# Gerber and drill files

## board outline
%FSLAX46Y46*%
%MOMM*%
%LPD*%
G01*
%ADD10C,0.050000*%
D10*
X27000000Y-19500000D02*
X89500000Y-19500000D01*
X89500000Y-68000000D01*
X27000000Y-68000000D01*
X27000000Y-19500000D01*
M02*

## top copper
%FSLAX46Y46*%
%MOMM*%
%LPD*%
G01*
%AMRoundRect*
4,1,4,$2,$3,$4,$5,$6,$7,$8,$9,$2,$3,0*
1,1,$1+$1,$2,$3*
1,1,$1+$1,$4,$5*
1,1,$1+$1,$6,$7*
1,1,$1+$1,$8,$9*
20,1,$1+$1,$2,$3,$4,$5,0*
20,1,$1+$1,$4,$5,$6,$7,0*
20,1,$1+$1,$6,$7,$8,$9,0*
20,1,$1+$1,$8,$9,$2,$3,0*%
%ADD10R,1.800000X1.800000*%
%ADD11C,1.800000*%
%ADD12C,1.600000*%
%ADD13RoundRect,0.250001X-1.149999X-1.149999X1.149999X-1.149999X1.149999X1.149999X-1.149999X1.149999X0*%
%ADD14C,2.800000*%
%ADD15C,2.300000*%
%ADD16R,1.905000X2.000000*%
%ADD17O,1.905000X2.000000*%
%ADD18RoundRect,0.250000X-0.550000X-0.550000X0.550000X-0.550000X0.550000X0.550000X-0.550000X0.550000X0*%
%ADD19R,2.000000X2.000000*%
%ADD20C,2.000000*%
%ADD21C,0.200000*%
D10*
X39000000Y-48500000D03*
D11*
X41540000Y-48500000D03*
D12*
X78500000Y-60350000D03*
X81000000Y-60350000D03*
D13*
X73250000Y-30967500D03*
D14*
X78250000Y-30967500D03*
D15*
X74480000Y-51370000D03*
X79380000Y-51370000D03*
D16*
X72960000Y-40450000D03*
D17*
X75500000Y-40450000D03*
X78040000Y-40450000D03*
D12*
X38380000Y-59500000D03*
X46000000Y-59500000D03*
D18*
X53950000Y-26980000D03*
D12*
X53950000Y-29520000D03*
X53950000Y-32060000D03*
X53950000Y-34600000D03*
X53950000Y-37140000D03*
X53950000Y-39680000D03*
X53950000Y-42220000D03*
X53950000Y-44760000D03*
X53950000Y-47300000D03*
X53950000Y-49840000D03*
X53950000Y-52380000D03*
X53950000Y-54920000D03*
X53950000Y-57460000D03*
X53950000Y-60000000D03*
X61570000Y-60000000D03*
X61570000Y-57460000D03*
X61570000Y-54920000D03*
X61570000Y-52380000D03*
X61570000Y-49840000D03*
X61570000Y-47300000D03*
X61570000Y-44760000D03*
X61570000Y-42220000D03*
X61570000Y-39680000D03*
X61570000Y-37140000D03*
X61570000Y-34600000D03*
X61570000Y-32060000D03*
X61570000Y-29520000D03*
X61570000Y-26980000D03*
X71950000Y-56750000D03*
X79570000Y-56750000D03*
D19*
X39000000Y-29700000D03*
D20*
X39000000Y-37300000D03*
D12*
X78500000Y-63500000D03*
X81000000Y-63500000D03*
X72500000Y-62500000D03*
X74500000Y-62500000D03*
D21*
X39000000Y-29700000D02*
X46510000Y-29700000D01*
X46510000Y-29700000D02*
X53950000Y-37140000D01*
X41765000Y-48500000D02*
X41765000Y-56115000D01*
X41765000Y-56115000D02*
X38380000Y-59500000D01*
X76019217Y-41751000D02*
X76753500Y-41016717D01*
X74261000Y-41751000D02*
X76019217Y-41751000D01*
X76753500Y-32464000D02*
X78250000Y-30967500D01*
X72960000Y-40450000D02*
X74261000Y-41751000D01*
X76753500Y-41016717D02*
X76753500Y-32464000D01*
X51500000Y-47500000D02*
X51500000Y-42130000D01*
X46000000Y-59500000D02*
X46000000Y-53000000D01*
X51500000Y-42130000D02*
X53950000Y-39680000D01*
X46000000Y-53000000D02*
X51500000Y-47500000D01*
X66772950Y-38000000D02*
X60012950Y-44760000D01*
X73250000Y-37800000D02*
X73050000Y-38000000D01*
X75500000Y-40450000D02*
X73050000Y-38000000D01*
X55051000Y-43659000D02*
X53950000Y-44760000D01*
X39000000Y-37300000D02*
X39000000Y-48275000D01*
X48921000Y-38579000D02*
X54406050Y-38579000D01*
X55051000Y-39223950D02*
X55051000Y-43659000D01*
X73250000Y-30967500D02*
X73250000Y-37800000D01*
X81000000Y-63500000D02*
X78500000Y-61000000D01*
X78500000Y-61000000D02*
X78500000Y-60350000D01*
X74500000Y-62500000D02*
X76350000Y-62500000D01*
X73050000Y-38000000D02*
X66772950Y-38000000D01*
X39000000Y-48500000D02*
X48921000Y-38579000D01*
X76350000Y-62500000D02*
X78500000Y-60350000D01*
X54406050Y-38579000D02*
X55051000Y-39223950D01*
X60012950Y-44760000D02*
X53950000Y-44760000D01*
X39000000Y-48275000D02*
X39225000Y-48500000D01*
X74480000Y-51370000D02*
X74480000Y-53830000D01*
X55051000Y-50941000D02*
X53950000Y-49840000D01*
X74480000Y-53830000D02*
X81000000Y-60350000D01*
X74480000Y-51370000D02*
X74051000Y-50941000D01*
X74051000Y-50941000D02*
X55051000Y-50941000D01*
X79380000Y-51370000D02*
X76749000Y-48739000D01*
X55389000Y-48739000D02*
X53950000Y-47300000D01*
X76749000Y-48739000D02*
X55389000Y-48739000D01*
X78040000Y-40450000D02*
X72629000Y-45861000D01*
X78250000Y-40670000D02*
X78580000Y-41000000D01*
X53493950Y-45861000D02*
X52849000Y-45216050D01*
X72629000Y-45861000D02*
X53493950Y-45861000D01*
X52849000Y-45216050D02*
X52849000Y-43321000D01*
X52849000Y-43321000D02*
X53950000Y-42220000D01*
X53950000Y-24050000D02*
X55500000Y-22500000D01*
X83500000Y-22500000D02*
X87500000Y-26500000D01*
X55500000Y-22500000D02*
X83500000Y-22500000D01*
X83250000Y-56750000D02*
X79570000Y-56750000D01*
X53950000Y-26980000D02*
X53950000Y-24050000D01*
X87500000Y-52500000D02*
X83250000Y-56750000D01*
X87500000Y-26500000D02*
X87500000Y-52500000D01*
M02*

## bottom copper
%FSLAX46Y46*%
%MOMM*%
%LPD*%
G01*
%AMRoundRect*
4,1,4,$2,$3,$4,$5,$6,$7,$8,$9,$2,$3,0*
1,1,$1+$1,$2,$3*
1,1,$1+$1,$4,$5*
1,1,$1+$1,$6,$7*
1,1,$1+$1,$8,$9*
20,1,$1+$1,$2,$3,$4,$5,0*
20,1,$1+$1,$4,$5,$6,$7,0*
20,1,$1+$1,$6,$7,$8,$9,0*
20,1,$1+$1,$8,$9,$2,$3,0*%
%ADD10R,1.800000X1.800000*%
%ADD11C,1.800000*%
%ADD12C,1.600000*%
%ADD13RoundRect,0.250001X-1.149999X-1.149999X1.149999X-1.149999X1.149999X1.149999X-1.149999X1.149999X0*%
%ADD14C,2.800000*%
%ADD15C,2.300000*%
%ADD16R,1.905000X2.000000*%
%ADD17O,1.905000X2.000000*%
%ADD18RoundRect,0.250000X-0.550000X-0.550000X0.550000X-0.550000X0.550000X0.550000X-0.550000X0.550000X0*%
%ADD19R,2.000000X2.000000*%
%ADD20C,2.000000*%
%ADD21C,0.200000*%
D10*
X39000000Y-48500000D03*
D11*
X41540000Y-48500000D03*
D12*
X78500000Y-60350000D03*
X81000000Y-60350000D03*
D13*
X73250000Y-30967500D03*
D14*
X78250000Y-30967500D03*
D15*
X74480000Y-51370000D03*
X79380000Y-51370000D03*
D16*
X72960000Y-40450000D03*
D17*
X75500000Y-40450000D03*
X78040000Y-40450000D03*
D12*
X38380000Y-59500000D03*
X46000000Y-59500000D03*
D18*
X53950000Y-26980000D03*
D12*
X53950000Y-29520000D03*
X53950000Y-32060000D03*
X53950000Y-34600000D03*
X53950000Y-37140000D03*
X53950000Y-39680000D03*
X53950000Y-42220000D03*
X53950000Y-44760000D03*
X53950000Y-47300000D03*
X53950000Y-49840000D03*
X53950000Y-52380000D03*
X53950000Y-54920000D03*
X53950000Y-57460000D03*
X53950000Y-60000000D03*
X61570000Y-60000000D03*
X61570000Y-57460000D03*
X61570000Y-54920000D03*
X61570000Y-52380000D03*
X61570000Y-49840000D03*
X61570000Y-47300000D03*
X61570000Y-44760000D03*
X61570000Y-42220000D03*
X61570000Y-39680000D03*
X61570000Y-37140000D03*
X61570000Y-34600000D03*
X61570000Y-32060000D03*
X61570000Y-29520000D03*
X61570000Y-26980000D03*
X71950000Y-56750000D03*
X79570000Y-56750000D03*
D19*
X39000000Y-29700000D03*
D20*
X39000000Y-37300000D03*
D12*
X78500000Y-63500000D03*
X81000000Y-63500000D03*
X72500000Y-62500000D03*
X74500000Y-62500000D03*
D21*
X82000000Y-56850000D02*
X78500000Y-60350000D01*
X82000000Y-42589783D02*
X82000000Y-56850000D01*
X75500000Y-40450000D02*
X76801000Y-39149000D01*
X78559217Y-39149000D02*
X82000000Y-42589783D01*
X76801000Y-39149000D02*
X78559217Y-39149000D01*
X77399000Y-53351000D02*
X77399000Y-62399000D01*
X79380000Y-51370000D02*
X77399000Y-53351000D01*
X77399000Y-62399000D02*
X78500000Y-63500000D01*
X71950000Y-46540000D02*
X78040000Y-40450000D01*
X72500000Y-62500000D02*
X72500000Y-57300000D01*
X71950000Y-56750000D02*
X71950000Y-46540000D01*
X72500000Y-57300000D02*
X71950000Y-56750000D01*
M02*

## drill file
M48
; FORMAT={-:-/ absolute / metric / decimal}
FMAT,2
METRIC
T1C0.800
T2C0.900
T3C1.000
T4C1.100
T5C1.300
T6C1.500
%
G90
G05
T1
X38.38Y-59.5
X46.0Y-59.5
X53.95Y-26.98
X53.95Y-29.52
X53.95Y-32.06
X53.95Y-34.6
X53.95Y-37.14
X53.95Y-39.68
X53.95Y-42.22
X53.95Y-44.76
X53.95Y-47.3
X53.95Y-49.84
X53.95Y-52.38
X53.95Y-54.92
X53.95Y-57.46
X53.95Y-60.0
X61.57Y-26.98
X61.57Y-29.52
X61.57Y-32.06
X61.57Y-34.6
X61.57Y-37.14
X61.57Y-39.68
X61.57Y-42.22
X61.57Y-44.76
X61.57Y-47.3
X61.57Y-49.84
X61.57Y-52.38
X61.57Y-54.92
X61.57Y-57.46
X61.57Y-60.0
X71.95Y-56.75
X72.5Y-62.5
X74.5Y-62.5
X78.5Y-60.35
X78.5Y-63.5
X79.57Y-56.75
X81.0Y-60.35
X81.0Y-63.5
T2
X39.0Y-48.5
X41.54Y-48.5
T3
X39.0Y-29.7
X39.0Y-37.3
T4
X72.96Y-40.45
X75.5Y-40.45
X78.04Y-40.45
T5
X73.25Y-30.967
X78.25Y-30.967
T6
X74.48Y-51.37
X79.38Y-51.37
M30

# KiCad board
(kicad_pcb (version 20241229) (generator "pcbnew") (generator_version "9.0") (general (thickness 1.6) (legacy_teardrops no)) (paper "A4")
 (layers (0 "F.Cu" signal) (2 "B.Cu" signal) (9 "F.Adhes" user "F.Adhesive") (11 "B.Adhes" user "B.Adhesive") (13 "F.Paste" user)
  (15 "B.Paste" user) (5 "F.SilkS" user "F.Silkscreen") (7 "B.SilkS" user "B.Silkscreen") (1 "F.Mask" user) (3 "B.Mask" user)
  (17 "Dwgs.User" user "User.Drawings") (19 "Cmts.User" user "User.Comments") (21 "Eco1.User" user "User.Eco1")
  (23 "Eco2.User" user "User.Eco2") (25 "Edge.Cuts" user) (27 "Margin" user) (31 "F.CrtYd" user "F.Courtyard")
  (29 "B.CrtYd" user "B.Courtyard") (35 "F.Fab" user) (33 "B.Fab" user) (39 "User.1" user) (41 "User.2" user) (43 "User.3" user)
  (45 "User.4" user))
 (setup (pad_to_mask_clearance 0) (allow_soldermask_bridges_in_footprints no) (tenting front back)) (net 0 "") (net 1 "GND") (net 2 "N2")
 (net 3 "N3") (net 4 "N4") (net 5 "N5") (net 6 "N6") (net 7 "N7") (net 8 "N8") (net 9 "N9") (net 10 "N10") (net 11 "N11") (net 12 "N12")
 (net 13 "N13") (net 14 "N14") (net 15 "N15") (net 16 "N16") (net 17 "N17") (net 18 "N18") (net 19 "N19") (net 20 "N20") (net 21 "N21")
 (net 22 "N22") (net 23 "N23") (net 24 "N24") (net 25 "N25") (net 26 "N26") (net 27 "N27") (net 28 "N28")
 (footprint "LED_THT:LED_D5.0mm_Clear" (layer "F.Cu") (at 39 48.5)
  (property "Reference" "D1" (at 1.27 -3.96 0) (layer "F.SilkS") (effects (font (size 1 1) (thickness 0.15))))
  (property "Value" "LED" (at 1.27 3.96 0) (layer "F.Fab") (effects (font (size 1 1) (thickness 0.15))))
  (pad "1" thru_hole rect (at 0 0) (size 1.8 1.8) (drill 0.9) (layers "*.Cu" "*.Mask") (remove_unused_layers no) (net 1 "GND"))
  (pad "2" thru_hole circle (at 2.54 0) (size 1.8 1.8) (drill 0.9) (layers "*.Cu" "*.Mask") (remove_unused_layers no) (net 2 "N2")))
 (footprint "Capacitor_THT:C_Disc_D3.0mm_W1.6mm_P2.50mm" (layer "F.Cu") (at 78.5 60.35)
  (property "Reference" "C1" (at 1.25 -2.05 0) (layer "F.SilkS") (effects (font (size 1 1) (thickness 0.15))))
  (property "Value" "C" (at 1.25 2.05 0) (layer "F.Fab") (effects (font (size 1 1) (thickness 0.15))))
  (pad "1" thru_hole circle (at 0 0) (size 1.6 1.6) (drill 0.8) (layers "*.Cu" "*.Mask") (remove_unused_layers no) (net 1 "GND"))
  (pad "2" thru_hole circle (at 2.5 0) (size 1.6 1.6) (drill 0.8) (layers "*.Cu" "*.Mask") (remove_unused_layers no) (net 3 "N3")))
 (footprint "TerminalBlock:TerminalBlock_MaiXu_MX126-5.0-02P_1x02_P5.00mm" (layer "F.Cu") (at 73.25 30.9675)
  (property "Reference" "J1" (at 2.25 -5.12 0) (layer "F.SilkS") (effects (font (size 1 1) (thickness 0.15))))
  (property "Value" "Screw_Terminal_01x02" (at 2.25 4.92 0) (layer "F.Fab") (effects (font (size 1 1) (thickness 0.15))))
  (pad "1" thru_hole roundrect (at 0 0) (size 2.8 2.8) (drill 1.3) (layers "*.Cu" "*.Mask") (remove_unused_layers no)
   (roundrect_rratio 0.089286) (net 1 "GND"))
  (pad "2" thru_hole circle (at 5 0) (size 2.8 2.8) (drill 1.3) (layers "*.Cu" "*.Mask") (remove_unused_layers no) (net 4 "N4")))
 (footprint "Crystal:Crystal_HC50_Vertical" (layer "F.Cu") (at 74.48 51.37)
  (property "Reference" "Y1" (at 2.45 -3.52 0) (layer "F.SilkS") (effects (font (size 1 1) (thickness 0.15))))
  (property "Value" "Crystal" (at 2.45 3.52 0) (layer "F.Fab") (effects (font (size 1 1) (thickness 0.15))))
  (pad "1" thru_hole circle (at 0 0) (size 2.3 2.3) (drill 1.5) (layers "*.Cu" "*.Mask") (remove_unused_layers no) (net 3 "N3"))
  (pad "2" thru_hole circle (at 4.9 0) (size 2.3 2.3) (drill 1.5) (layers "*.Cu" "*.Mask") (remove_unused_layers no) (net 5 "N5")))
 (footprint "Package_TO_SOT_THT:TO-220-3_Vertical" (layer "F.Cu") (at 72.96 40.45)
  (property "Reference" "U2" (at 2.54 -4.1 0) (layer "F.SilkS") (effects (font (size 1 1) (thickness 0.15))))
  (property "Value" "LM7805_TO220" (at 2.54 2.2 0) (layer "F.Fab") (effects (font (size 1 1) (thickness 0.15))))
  (pad "1" thru_hole rect (at 0 0) (size 1.905 2) (drill 1.1) (layers "*.Cu" "*.Mask") (remove_unused_layers no) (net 4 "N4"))
  (pad "2" thru_hole oval (at 2.54 0) (size 1.905 2) (drill 1.1) (layers "*.Cu" "*.Mask") (remove_unused_layers no) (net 1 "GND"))
  (pad "3" thru_hole oval (at 5.08 0) (size 1.905 2) (drill 1.1) (layers "*.Cu" "*.Mask") (remove_unused_layers no) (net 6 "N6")))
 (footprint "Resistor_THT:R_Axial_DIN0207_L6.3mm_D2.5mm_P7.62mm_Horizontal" (layer "F.Cu") (at 38.38 59.5)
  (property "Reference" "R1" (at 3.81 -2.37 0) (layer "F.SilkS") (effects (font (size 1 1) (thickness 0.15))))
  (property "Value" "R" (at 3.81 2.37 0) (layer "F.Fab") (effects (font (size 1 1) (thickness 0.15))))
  (pad "1" thru_hole circle (at 0 0) (size 1.6 1.6) (drill 0.8) (layers "*.Cu" "*.Mask") (remove_unused_layers no) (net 2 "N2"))
  (pad "2" thru_hole circle (at 7.62 0) (size 1.6 1.6) (drill 0.8) (layers "*.Cu" "*.Mask") (remove_unused_layers no) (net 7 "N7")))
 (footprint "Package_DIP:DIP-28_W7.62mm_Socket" (layer "F.Cu") (at 53.95 26.98)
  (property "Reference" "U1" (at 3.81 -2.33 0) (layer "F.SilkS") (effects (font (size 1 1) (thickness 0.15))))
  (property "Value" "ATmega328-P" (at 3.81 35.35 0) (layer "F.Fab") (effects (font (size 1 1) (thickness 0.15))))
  (pad "1" thru_hole roundrect (at 0 0) (size 1.6 1.6) (drill 0.8) (layers "*.Cu" "*.Mask") (remove_unused_layers no)
   (roundrect_rratio 0.15625) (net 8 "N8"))
  (pad "2" thru_hole circle (at 0 2.54) (size 1.6 1.6) (drill 0.8) (layers "*.Cu" "*.Mask") (remove_unused_layers no) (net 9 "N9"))
  (pad "3" thru_hole circle (at 0 5.08) (size 1.6 1.6) (drill 0.8) (layers "*.Cu" "*.Mask") (remove_unused_layers no) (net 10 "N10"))
  (pad "4" thru_hole circle (at 0 7.62) (size 1.6 1.6) (drill 0.8) (layers "*.Cu" "*.Mask") (remove_unused_layers no) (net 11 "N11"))
  (pad "5" thru_hole circle (at 0 10.16) (size 1.6 1.6) (drill 0.8) (layers "*.Cu" "*.Mask") (remove_unused_layers no) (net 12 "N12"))
  (pad "6" thru_hole circle (at 0 12.7) (size 1.6 1.6) (drill 0.8) (layers "*.Cu" "*.Mask") (remove_unused_layers no) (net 7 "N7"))
  (pad "7" thru_hole circle (at 0 15.24) (size 1.6 1.6) (drill 0.8) (layers "*.Cu" "*.Mask") (remove_unused_layers no) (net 6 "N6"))
  (pad "8" thru_hole circle (at 0 17.78) (size 1.6 1.6) (drill 0.8) (layers "*.Cu" "*.Mask") (remove_unused_layers no) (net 1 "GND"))
  (pad "9" thru_hole circle (at 0 20.32) (size 1.6 1.6) (drill 0.8) (layers "*.Cu" "*.Mask") (remove_unused_layers no) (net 5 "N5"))
  (pad "10" thru_hole circle (at 0 22.86) (size 1.6 1.6) (drill 0.8) (layers "*.Cu" "*.Mask") (remove_unused_layers no) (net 3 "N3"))
  (pad "11" thru_hole circle (at 0 25.4) (size 1.6 1.6) (drill 0.8) (layers "*.Cu" "*.Mask") (remove_unused_layers no) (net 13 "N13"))
  (pad "12" thru_hole circle (at 0 27.94) (size 1.6 1.6) (drill 0.8) (layers "*.Cu" "*.Mask") (remove_unused_layers no) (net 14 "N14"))
  (pad "13" thru_hole circle (at 0 30.48) (size 1.6 1.6) (drill 0.8) (layers "*.Cu" "*.Mask") (remove_unused_layers no) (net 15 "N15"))
  (pad "14" thru_hole circle (at 0 33.02) (size 1.6 1.6) (drill 0.8) (layers "*.Cu" "*.Mask") (remove_unused_layers no) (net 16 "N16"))
  (pad "15" thru_hole circle (at 7.62 33.02) (size 1.6 1.6) (drill 0.8) (layers "*.Cu" "*.Mask") (remove_unused_layers no) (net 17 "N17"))
  (pad "16" thru_hole circle (at 7.62 30.48) (size 1.6 1.6) (drill 0.8) (layers "*.Cu" "*.Mask") (remove_unused_layers no) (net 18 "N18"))
  (pad "17" thru_hole circle (at 7.62 27.94) (size 1.6 1.6) (drill 0.8) (layers "*.Cu" "*.Mask") (remove_unused_layers no) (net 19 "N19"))
  (pad "18" thru_hole circle (at 7.62 25.4) (size 1.6 1.6) (drill 0.8) (layers "*.Cu" "*.Mask") (remove_unused_layers no) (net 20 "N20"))
  (pad "19" thru_hole circle (at 7.62 22.86) (size 1.6 1.6) (drill 0.8) (layers "*.Cu" "*.Mask") (remove_unused_layers no) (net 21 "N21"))
  (pad "20" thru_hole circle (at 7.62 20.32) (size 1.6 1.6) (drill 0.8) (layers "*.Cu" "*.Mask") (remove_unused_layers no) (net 6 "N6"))
  (pad "21" thru_hole circle (at 7.62 17.78) (size 1.6 1.6) (drill 0.8) (layers "*.Cu" "*.Mask") (remove_unused_layers no) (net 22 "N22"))
  (pad "22" thru_hole circle (at 7.62 15.24) (size 1.6 1.6) (drill 0.8) (layers "*.Cu" "*.Mask") (remove_unused_layers no) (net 1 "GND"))
  (pad "23" thru_hole circle (at 7.62 12.7) (size 1.6 1.6) (drill 0.8) (layers "*.Cu" "*.Mask") (remove_unused_layers no) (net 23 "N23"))
  (pad "24" thru_hole circle (at 7.62 10.16) (size 1.6 1.6) (drill 0.8) (layers "*.Cu" "*.Mask") (remove_unused_layers no) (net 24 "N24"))
  (pad "25" thru_hole circle (at 7.62 7.62) (size 1.6 1.6) (drill 0.8) (layers "*.Cu" "*.Mask") (remove_unused_layers no) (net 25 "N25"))
  (pad "26" thru_hole circle (at 7.62 5.08) (size 1.6 1.6) (drill 0.8) (layers "*.Cu" "*.Mask") (remove_unused_layers no) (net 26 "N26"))
  (pad "27" thru_hole circle (at 7.62 2.54) (size 1.6 1.6) (drill 0.8) (layers "*.Cu" "*.Mask") (remove_unused_layers no) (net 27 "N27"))
  (pad "28" thru_hole circle (at 7.62 0) (size 1.6 1.6) (drill 0.8) (layers "*.Cu" "*.Mask") (remove_unused_layers no) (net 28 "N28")))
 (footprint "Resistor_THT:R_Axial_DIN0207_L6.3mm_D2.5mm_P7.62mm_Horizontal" (layer "F.Cu") (at 71.95 56.75)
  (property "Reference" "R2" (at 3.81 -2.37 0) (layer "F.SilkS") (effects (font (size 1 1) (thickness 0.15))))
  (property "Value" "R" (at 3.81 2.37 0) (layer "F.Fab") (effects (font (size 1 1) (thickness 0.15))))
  (pad "1" thru_hole circle (at 0 0) (size 1.6 1.6) (drill 0.8) (layers "*.Cu" "*.Mask") (remove_unused_layers no) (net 6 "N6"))
  (pad "2" thru_hole circle (at 7.62 0) (size 1.6 1.6) (drill 0.8) (layers "*.Cu" "*.Mask") (remove_unused_layers no) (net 8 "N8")))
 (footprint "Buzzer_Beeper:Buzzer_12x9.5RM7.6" (layer "F.Cu") (at 39 29.7 -90)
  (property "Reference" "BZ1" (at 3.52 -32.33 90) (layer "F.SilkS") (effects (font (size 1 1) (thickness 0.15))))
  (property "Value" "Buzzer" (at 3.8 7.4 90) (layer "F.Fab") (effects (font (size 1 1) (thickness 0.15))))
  (pad "1" thru_hole rect (at 0 0 270) (size 2 2) (drill 1) (layers "*.Cu" "*.Mask") (remove_unused_layers no) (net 12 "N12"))
  (pad "2" thru_hole circle (at 7.6 0 270) (size 2 2) (drill 1) (layers "*.Cu" "*.Mask") (remove_unused_layers no) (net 1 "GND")))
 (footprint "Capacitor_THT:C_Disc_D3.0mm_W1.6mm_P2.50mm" (layer "F.Cu") (at 78.5 63.5)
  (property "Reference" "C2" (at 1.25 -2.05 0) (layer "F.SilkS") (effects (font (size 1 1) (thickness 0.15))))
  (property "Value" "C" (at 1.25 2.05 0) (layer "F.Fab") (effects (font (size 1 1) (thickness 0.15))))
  (pad "1" thru_hole circle (at 0 0) (size 1.6 1.6) (drill 0.8) (layers "*.Cu" "*.Mask") (remove_unused_layers no) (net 5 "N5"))
  (pad "2" thru_hole circle (at 2.5 0) (size 1.6 1.6) (drill 0.8) (layers "*.Cu" "*.Mask") (remove_unused_layers no) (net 1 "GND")))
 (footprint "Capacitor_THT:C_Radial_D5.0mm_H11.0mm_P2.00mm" (layer "F.Cu") (at 72.5 62.5)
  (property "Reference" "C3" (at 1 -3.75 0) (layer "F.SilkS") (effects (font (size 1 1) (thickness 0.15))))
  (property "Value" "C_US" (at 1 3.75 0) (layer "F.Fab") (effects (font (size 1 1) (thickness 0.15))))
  (pad "1" thru_hole circle (at 0 0) (size 1.6 1.6) (drill 0.8) (layers "*.Cu" "*.Mask") (remove_unused_layers no) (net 6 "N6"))
  (pad "2" thru_hole circle (at 2 0) (size 1.6 1.6) (drill 0.8) (layers "*.Cu" "*.Mask") (remove_unused_layers no) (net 1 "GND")))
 (gr_rect (start 27 19.5) (end 89.5 68) (stroke (width 0.05) (type default)) (fill no) (layer "Edge.Cuts"))
 (segment (start 39 29.7) (end 46.51 29.7) (width 0.2) (layer "F.Cu") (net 12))
 (segment (start 46.51 29.7) (end 53.95 37.14) (width 0.2) (layer "F.Cu") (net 12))
 (segment (start 41.765 48.5) (end 41.765 56.115) (width 0.2) (layer "F.Cu") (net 2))
 (segment (start 41.765 56.115) (end 38.38 59.5) (width 0.2) (layer "F.Cu") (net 2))
 (segment (start 76.019217 41.751) (end 76.7535 41.016717) (width 0.2) (layer "F.Cu") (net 4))
 (segment (start 74.261 41.751) (end 76.019217 41.751) (width 0.2) (layer "F.Cu") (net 4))
 (segment (start 76.7535 32.464) (end 78.25 30.9675) (width 0.2) (layer "F.Cu") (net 4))
 (segment (start 72.96 40.45) (end 74.261 41.751) (width 0.2) (layer "F.Cu") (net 4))
 (segment (start 76.7535 41.016717) (end 76.7535 32.464) (width 0.2) (layer "F.Cu") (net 4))
 (segment (start 51.5 47.5) (end 51.5 42.13) (width 0.2) (layer "F.Cu") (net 7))
 (segment (start 46 59.5) (end 46 53) (width 0.2) (layer "F.Cu") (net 7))
 (segment (start 51.5 42.13) (end 53.95 39.68) (width 0.2) (layer "F.Cu") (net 7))
 (segment (start 46 53) (end 51.5 47.5) (width 0.2) (layer "F.Cu") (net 7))
 (segment (start 66.77295 38) (end 60.01295 44.76) (width 0.2) (layer "F.Cu") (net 1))
 (segment (start 73.25 37.8) (end 73.05 38) (width 0.2) (layer "F.Cu") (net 1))
 (segment (start 75.5 40.45) (end 73.05 38) (width 0.2) (layer "F.Cu") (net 1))
 (segment (start 55.051 43.659) (end 53.95 44.76) (width 0.2) (layer "F.Cu") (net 1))
 (segment (start 39 37.3) (end 39 48.275) (width 0.2) (layer "F.Cu") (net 1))
 (segment (start 48.921 38.579) (end 54.40605 38.579) (width 0.2) (layer "F.Cu") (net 1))
 (segment (start 55.051 39.22395) (end 55.051 43.659) (width 0.2) (layer "F.Cu") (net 1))
 (segment (start 73.25 30.9675) (end 73.25 37.8) (width 0.2) (layer "F.Cu") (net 1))
 (segment (start 81 63.5) (end 78.5 61) (width 0.2) (layer "F.Cu") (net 1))
 (segment (start 78.5 61) (end 78.5 60.35) (width 0.2) (layer "F.Cu") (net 1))
 (segment (start 74.5 62.5) (end 76.35 62.5) (width 0.2) (layer "F.Cu") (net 1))
 (segment (start 73.05 38) (end 66.77295 38) (width 0.2) (layer "F.Cu") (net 1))
 (segment (start 39 48.5) (end 48.921 38.579) (width 0.2) (layer "F.Cu") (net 1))
 (segment (start 76.35 62.5) (end 78.5 60.35) (width 0.2) (layer "F.Cu") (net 1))
 (segment (start 54.40605 38.579) (end 55.051 39.22395) (width 0.2) (layer "F.Cu") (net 1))
 (segment (start 60.01295 44.76) (end 53.95 44.76) (width 0.2) (layer "F.Cu") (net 1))
 (segment (start 39 48.275) (end 39.225 48.5) (width 0.2) (layer "F.Cu") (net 1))
 (segment (start 82 56.85) (end 78.5 60.35) (width 0.2) (layer "B.Cu") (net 1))
 (segment (start 82 42.589783) (end 82 56.85) (width 0.2) (layer "B.Cu") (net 1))
 (segment (start 75.5 40.45) (end 76.801 39.149) (width 0.2) (layer "B.Cu") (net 1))
 (segment (start 78.559217 39.149) (end 82 42.589783) (width 0.2) (layer "B.Cu") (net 1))
 (segment (start 76.801 39.149) (end 78.559217 39.149) (width 0.2) (layer "B.Cu") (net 1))
 (segment (start 74.48 51.37) (end 74.48 53.83) (width 0.2) (layer "F.Cu") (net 3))
 (segment (start 55.051 50.941) (end 53.95 49.84) (width 0.2) (layer "F.Cu") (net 3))
 (segment (start 74.48 53.83) (end 81 60.35) (width 0.2) (layer "F.Cu") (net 3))
 (segment (start 74.48 51.37) (end 74.051 50.941) (width 0.2) (layer "F.Cu") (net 3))
 (segment (start 74.051 50.941) (end 55.051 50.941) (width 0.2) (layer "F.Cu") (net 3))
 (segment (start 79.38 51.37) (end 76.749 48.739) (width 0.2) (layer "F.Cu") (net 5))
 (segment (start 55.389 48.739) (end 53.95 47.3) (width 0.2) (layer "F.Cu") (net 5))
 (segment (start 76.749 48.739) (end 55.389 48.739) (width 0.2) (layer "F.Cu") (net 5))
 (segment (start 77.399 53.351) (end 77.399 62.399) (width 0.2) (layer "B.Cu") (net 5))
 (segment (start 79.38 51.37) (end 77.399 53.351) (width 0.2) (layer "B.Cu") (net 5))
 (segment (start 77.399 62.399) (end 78.5 63.5) (width 0.2) (layer "B.Cu") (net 5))
 (segment (start 78.04 40.45) (end 72.629 45.861) (width 0.2) (layer "F.Cu") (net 6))
 (segment (start 78.25 40.67) (end 78.58 41) (width 0.2) (layer "F.Cu") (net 6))
 (segment (start 53.49395 45.861) (end 52.849 45.21605) (width 0.2) (layer "F.Cu") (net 6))
 (segment (start 72.629 45.861) (end 53.49395 45.861) (width 0.2) (layer "F.Cu") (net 6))
 (segment (start 52.849 45.21605) (end 52.849 43.321) (width 0.2) (layer "F.Cu") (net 6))
 (segment (start 52.849 43.321) (end 53.95 42.22) (width 0.2) (layer "F.Cu") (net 6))
 (segment (start 71.95 46.54) (end 78.04 40.45) (width 0.2) (layer "B.Cu") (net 6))
 (segment (start 72.5 62.5) (end 72.5 57.3) (width 0.2) (layer "B.Cu") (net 6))
 (segment (start 71.95 56.75) (end 71.95 46.54) (width 0.2) (layer "B.Cu") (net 6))
 (segment (start 72.5 57.3) (end 71.95 56.75) (width 0.2) (layer "B.Cu") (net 6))
 (segment (start 53.95 24.05) (end 55.5 22.5) (width 0.2) (layer "F.Cu") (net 8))
 (segment (start 83.5 22.5) (end 87.5 26.5) (width 0.2) (layer "F.Cu") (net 8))
 (segment (start 55.5 22.5) (end 83.5 22.5) (width 0.2) (layer "F.Cu") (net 8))
 (segment (start 83.25 56.75) (end 79.57 56.75) (width 0.2) (layer "F.Cu") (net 8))
 (segment (start 53.95 26.98) (end 53.95 24.05) (width 0.2) (layer "F.Cu") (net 8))
 (segment (start 87.5 52.5) (end 83.25 56.75) (width 0.2) (layer "F.Cu") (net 8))
 (segment (start 87.5 26.5) (end 87.5 52.5) (width 0.2) (layer "F.Cu") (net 8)))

